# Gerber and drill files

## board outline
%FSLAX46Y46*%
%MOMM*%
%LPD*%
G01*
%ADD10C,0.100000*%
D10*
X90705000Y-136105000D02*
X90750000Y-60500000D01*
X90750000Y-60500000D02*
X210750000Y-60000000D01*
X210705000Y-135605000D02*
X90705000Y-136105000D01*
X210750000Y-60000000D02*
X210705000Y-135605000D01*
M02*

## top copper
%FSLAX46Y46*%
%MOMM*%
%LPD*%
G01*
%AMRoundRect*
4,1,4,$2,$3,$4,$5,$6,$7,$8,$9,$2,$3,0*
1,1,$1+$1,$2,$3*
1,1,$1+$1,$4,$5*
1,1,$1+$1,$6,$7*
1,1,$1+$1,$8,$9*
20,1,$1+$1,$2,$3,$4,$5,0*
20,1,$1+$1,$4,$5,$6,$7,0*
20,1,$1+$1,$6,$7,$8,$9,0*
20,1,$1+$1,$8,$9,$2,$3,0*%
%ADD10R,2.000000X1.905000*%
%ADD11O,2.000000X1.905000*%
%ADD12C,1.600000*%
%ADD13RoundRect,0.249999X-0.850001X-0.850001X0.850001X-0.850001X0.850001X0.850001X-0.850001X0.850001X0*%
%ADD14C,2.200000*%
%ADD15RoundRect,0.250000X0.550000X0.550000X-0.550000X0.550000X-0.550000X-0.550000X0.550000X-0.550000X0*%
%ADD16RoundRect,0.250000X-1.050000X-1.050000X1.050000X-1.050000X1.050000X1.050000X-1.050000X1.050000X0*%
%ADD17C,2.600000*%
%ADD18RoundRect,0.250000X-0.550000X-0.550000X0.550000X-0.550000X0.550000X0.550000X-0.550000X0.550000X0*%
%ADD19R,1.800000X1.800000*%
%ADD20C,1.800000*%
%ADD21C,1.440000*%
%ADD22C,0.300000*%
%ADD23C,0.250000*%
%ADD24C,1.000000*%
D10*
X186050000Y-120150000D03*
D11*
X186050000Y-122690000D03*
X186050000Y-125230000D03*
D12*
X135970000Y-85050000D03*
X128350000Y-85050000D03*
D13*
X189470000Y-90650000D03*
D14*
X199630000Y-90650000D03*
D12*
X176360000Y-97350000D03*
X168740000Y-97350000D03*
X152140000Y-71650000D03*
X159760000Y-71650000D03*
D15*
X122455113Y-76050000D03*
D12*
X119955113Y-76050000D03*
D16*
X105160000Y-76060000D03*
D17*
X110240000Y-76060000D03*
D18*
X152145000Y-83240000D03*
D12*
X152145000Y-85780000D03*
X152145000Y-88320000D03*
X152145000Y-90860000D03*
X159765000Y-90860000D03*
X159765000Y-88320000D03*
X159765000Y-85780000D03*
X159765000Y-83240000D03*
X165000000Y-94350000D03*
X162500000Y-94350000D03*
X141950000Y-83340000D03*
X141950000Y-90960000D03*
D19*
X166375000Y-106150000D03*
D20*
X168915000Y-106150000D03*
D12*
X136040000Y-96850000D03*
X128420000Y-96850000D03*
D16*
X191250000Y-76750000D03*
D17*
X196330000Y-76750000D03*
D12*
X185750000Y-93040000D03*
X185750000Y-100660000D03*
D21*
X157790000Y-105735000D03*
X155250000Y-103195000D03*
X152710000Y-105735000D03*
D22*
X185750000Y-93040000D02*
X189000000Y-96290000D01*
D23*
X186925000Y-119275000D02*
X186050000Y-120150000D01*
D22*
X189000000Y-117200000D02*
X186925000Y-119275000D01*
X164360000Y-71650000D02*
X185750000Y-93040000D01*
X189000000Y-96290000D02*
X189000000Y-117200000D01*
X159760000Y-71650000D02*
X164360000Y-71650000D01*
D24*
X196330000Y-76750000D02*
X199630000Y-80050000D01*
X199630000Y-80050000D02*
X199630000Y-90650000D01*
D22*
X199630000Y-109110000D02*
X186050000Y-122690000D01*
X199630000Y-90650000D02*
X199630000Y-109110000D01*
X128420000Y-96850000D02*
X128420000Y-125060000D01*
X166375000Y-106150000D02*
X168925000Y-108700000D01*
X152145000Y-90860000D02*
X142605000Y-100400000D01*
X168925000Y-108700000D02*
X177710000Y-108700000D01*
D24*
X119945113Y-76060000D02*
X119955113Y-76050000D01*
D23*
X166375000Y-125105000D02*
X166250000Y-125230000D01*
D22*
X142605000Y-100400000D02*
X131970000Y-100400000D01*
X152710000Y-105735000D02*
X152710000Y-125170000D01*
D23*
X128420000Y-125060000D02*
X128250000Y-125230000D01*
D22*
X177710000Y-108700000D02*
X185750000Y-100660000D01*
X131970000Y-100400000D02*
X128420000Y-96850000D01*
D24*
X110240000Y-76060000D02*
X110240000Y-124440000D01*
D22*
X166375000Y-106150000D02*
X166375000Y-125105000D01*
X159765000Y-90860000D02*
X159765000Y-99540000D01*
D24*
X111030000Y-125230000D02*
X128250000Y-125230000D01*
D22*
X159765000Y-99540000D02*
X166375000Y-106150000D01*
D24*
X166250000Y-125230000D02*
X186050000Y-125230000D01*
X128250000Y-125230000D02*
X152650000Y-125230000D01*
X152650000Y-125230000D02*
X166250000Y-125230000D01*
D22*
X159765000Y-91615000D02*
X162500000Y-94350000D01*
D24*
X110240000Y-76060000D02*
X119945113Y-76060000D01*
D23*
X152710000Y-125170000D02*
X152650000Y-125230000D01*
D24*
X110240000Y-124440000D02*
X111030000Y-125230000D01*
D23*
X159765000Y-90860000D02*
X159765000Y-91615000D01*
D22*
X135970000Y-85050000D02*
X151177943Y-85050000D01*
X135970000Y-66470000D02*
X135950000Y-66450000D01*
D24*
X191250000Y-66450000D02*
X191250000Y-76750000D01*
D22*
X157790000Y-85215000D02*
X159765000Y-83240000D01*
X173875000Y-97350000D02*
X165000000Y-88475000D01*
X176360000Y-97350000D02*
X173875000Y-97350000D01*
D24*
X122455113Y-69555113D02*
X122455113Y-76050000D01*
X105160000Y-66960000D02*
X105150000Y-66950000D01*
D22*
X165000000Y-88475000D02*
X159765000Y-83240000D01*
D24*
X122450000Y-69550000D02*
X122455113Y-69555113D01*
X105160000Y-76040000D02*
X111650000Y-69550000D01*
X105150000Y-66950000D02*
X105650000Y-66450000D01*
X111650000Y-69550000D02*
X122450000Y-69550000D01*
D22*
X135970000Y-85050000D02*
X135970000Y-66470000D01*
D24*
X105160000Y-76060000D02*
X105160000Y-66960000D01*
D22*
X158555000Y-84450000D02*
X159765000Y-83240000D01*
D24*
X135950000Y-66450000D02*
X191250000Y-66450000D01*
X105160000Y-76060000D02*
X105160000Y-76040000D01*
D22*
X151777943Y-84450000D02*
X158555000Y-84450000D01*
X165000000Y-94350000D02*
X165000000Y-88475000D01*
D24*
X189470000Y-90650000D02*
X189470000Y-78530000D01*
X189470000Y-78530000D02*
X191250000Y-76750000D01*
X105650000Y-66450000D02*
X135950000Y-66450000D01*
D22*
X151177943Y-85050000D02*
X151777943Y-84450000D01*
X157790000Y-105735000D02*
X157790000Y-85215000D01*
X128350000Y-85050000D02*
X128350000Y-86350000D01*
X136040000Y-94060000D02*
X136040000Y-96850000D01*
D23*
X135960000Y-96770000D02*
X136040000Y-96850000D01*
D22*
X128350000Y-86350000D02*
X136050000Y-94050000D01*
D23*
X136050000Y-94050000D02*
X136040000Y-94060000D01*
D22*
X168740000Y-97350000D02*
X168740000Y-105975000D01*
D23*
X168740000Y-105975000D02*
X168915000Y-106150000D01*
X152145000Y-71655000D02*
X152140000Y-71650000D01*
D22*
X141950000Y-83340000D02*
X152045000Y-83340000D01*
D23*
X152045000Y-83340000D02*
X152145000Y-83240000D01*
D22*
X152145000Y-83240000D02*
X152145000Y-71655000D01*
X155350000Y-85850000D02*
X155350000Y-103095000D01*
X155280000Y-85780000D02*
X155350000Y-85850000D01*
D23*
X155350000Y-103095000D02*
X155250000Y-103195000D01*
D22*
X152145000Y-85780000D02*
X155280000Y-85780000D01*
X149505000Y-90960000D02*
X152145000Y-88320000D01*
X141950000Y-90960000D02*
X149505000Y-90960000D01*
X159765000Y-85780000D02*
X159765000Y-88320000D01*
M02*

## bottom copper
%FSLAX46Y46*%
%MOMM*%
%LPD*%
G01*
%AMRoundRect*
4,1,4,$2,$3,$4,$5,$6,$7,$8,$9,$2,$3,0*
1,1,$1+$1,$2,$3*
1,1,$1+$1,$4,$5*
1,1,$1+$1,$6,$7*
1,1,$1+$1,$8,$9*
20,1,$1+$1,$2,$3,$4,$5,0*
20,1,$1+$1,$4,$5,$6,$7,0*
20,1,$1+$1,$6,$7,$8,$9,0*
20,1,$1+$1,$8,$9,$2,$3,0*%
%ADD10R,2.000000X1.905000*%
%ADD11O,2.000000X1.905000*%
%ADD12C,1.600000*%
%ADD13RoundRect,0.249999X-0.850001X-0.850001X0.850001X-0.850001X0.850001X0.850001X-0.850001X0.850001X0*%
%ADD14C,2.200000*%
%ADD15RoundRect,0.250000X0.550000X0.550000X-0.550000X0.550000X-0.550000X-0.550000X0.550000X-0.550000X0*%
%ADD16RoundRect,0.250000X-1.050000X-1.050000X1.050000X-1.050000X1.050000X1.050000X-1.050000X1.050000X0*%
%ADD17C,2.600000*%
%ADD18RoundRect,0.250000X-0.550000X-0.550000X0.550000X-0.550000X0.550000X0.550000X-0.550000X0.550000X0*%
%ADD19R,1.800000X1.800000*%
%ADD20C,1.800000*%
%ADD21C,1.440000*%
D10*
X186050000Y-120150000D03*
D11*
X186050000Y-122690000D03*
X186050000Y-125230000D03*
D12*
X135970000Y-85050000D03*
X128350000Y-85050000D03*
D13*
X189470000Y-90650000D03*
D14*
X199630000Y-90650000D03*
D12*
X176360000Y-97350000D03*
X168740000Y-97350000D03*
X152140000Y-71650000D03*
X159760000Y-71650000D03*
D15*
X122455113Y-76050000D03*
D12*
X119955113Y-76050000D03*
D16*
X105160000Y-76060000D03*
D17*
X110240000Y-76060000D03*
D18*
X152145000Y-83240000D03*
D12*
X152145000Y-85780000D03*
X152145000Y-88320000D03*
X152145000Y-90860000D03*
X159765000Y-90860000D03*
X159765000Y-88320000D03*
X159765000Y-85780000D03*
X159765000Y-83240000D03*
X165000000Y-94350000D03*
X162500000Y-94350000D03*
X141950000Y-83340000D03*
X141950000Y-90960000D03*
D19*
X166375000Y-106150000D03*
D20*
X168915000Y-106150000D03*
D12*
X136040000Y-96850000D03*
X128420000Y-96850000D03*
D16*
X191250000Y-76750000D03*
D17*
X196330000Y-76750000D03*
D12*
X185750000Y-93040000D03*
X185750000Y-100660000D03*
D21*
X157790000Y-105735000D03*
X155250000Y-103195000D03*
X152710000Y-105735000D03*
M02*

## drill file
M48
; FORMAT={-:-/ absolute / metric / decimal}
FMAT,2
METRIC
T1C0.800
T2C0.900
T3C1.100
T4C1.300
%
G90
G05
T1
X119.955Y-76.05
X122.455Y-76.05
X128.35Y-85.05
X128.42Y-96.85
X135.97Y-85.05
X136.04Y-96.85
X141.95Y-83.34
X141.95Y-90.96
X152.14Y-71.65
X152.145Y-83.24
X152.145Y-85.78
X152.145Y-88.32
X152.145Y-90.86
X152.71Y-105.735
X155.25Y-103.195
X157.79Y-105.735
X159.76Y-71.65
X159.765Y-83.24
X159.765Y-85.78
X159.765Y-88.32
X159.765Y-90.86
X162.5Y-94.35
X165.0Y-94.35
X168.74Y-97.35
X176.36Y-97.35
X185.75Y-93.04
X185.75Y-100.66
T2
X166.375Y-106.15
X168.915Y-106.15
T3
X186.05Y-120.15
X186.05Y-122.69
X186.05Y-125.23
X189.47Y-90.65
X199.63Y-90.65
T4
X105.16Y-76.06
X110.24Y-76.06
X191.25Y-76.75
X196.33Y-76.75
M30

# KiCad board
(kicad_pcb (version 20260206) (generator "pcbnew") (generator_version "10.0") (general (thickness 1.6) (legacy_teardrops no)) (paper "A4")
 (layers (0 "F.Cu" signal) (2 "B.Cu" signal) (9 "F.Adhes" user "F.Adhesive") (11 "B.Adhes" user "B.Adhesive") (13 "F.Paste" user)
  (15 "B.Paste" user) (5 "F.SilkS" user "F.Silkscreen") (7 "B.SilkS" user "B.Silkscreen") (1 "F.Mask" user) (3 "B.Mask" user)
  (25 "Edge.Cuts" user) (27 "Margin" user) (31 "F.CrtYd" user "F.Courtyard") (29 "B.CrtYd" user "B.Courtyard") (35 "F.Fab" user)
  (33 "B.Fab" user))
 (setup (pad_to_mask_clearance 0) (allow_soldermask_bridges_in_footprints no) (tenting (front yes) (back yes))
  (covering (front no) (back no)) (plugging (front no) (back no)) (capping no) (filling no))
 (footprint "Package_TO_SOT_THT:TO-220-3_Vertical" (layer "F.Cu") (at 186.05 120.15 -90)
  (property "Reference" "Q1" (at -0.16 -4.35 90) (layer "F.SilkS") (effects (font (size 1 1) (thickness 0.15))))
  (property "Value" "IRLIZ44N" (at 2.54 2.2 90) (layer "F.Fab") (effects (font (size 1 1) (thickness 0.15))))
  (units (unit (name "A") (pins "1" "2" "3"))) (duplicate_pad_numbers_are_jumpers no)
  (pad "1" thru_hole rect (at 0 0 270) (size 1.905 2) (drill 1.1) (layers "*.Cu" "*.Mask") (remove_unused_layers no) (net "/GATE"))
  (pad "2" thru_hole oval (at 2.54 0 270) (size 1.905 2) (drill 1.1) (layers "*.Cu" "*.Mask") (remove_unused_layers no) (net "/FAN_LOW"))
  (pad "3" thru_hole oval (at 5.08 0 270) (size 1.905 2) (drill 1.1) (layers "*.Cu" "*.Mask") (remove_unused_layers no) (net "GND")))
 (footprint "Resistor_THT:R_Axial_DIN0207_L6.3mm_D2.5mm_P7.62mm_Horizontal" (layer "F.Cu") (at 135.97 85.05 180)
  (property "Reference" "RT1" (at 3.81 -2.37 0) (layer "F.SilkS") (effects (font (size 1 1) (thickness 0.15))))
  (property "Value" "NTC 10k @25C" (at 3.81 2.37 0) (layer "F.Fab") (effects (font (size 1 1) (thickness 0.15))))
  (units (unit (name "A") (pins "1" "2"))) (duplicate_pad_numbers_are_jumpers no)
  (pad "1" thru_hole circle (at 0 0 180) (size 1.6 1.6) (drill 0.8) (layers "*.Cu" "*.Mask") (remove_unused_layers no) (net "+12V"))
  (pad "2" thru_hole circle (at 7.62 0 180) (size 1.6 1.6) (drill 0.8) (layers "*.Cu" "*.Mask") (remove_unused_layers no)
   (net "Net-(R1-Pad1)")))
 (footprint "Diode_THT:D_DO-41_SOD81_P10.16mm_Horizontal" (layer "F.Cu") (at 189.47 90.65)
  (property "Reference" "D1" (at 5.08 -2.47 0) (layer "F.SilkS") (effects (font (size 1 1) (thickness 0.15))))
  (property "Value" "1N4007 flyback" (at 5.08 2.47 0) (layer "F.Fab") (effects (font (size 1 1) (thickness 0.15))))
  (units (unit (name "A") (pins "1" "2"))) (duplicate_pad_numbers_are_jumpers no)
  (pad "1" thru_hole roundrect (at 0 0) (size 2.2 2.2) (drill 1.1) (layers "*.Cu" "*.Mask") (remove_unused_layers no)
   (roundrect_rratio 0.113636) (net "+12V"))
  (pad "2" thru_hole circle (at 10.16 0) (size 2.2 2.2) (drill 1.1) (layers "*.Cu" "*.Mask") (remove_unused_layers no) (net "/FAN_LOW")))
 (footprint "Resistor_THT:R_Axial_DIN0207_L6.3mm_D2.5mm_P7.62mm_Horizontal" (layer "F.Cu") (at 176.36 97.35 180)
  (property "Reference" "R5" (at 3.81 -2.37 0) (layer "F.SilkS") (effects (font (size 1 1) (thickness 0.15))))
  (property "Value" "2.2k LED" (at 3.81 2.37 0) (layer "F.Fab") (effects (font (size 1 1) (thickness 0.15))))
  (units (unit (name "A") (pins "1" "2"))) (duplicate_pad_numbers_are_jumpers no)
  (pad "1" thru_hole circle (at 0 0 180) (size 1.6 1.6) (drill 0.8) (layers "*.Cu" "*.Mask") (remove_unused_layers no) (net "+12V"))
  (pad "2" thru_hole circle (at 7.62 0 180) (size 1.6 1.6) (drill 0.8) (layers "*.Cu" "*.Mask") (remove_unused_layers no) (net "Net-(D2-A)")))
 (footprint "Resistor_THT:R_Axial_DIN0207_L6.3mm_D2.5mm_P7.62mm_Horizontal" (layer "F.Cu") (at 152.14 71.65)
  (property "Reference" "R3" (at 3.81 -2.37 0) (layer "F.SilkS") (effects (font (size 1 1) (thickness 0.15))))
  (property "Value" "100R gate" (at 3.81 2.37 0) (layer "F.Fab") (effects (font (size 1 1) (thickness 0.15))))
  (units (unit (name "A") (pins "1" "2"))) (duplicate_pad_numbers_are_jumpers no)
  (pad "1" thru_hole circle (at 0 0) (size 1.6 1.6) (drill 0.8) (layers "*.Cu" "*.Mask") (remove_unused_layers no) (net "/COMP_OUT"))
  (pad "2" thru_hole circle (at 7.62 0) (size 1.6 1.6) (drill 0.8) (layers "*.Cu" "*.Mask") (remove_unused_layers no) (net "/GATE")))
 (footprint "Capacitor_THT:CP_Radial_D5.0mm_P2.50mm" (layer "F.Cu") (at 122.455113 76.05 180)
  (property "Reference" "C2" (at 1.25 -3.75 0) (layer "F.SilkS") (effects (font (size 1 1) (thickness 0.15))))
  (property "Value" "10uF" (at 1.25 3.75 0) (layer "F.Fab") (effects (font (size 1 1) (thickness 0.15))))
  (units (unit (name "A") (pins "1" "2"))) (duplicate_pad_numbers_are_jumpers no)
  (pad "1" thru_hole roundrect (at 0 0 180) (size 1.6 1.6) (drill 0.8) (layers "*.Cu" "*.Mask") (remove_unused_layers no)
   (roundrect_rratio 0.15625) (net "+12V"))
  (pad "2" thru_hole circle (at 2.5 0 180) (size 1.6 1.6) (drill 0.8) (layers "*.Cu" "*.Mask") (remove_unused_layers no) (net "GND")))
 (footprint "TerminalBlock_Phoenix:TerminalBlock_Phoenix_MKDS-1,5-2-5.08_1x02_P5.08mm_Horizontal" (layer "F.Cu") (at 105.16 76.06)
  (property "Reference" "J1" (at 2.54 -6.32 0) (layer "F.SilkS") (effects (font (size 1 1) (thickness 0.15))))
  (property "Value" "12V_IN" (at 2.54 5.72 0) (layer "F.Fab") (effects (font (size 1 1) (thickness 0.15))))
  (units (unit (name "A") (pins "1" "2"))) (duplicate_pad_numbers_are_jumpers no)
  (pad "1" thru_hole roundrect (at 0 0) (size 2.6 2.6) (drill 1.3) (layers "*.Cu" "*.Mask") (remove_unused_layers no)
   (roundrect_rratio 0.096154) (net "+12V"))
  (pad "2" thru_hole circle (at 5.08 0) (size 2.6 2.6) (drill 1.3) (layers "*.Cu" "*.Mask") (remove_unused_layers no) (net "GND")))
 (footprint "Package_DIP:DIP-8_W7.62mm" (layer "F.Cu") (at 152.145 83.24)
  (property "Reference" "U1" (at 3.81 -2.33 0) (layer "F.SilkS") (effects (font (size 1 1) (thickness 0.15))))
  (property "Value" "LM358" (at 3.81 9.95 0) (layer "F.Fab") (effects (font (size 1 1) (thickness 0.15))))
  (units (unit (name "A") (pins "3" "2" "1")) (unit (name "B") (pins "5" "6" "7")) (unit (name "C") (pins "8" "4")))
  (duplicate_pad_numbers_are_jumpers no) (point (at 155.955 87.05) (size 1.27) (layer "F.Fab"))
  (pad "1" thru_hole roundrect (at 0 0) (size 1.6 1.6) (drill 0.8) (layers "*.Cu" "*.Mask") (remove_unused_layers no)
   (roundrect_rratio 0.15625) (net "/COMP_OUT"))
  (pad "2" thru_hole circle (at 0 2.54) (size 1.6 1.6) (drill 0.8) (layers "*.Cu" "*.Mask") (remove_unused_layers no) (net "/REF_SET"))
  (pad "3" thru_hole circle (at 0 5.08) (size 1.6 1.6) (drill 0.8) (layers "*.Cu" "*.Mask") (remove_unused_layers no) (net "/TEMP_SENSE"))
  (pad "4" thru_hole circle (at 0 7.62) (size 1.6 1.6) (drill 0.8) (layers "*.Cu" "*.Mask") (remove_unused_layers no) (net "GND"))
  (pad "5" thru_hole circle (at 7.62 7.62) (size 1.6 1.6) (drill 0.8) (layers "*.Cu" "*.Mask") (remove_unused_layers no) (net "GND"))
  (pad "6" thru_hole circle (at 7.62 5.08) (size 1.6 1.6) (drill 0.8) (layers "*.Cu" "*.Mask") (remove_unused_layers no) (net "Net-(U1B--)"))
  (pad "7" thru_hole circle (at 7.62 2.54) (size 1.6 1.6) (drill 0.8) (layers "*.Cu" "*.Mask") (remove_unused_layers no) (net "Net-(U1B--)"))
  (pad "8" thru_hole circle (at 7.62 0) (size 1.6 1.6) (drill 0.8) (layers "*.Cu" "*.Mask") (remove_unused_layers no) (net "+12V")))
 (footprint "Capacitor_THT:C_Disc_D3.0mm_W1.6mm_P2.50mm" (layer "F.Cu") (at 165 94.35 180)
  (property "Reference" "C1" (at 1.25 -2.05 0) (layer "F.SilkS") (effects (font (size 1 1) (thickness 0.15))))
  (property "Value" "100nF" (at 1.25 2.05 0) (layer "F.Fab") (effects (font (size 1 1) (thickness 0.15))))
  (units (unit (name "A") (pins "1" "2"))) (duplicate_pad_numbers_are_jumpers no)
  (pad "1" thru_hole circle (at 0 0 180) (size 1.6 1.6) (drill 0.8) (layers "*.Cu" "*.Mask") (remove_unused_layers no) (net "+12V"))
  (pad "2" thru_hole circle (at 2.5 0 180) (size 1.6 1.6) (drill 0.8) (layers "*.Cu" "*.Mask") (remove_unused_layers no) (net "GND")))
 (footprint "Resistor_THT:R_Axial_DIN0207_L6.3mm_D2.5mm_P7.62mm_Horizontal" (layer "F.Cu") (at 141.95 83.34 -90)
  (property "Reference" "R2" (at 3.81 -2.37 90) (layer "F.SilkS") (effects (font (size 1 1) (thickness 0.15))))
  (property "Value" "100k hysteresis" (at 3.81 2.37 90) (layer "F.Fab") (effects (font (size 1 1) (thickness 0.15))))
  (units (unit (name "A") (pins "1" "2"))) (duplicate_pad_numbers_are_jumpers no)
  (pad "1" thru_hole circle (at 0 0 270) (size 1.6 1.6) (drill 0.8) (layers "*.Cu" "*.Mask") (remove_unused_layers no) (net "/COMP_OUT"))
  (pad "2" thru_hole circle (at 7.62 0 270) (size 1.6 1.6) (drill 0.8) (layers "*.Cu" "*.Mask") (remove_unused_layers no)
   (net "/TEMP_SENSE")))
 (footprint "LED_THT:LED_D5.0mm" (layer "F.Cu") (at 166.375 106.15)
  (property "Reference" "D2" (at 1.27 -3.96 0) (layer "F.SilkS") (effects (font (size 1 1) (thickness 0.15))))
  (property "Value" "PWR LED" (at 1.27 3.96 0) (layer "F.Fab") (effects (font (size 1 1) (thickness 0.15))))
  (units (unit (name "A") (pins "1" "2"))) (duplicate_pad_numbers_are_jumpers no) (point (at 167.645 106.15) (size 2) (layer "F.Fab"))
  (pad "1" thru_hole rect (at 0 0) (size 1.8 1.8) (drill 0.9) (layers "*.Cu" "*.Mask") (remove_unused_layers no) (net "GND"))
  (pad "2" thru_hole circle (at 2.54 0) (size 1.8 1.8) (drill 0.9) (layers "*.Cu" "*.Mask") (remove_unused_layers no) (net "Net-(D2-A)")))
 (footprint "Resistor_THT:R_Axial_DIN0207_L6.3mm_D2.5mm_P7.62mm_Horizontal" (layer "F.Cu") (at 136.04 96.85 180)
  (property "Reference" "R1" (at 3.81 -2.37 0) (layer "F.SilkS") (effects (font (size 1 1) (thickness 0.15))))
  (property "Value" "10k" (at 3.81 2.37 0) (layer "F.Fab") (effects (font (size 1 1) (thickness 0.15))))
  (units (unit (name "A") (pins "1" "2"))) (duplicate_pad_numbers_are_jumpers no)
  (pad "1" thru_hole circle (at 0 0 180) (size 1.6 1.6) (drill 0.8) (layers "*.Cu" "*.Mask") (remove_unused_layers no) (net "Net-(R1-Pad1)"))
  (pad "2" thru_hole circle (at 7.62 0 180) (size 1.6 1.6) (drill 0.8) (layers "*.Cu" "*.Mask") (remove_unused_layers no) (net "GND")))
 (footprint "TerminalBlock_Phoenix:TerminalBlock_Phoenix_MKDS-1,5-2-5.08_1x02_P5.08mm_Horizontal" (layer "F.Cu") (at 191.25 76.75)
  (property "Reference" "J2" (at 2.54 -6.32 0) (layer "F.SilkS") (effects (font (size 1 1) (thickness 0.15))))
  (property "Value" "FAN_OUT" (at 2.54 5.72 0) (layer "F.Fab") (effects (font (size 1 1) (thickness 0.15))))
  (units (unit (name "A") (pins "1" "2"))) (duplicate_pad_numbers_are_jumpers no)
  (pad "1" thru_hole roundrect (at 0 0) (size 2.6 2.6) (drill 1.3) (layers "*.Cu" "*.Mask") (remove_unused_layers no)
   (roundrect_rratio 0.096154) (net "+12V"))
  (pad "2" thru_hole circle (at 5.08 0) (size 2.6 2.6) (drill 1.3) (layers "*.Cu" "*.Mask") (remove_unused_layers no) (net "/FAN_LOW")))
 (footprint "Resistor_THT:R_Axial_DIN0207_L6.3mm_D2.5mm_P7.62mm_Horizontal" (layer "F.Cu") (at 185.75 93.04 -90)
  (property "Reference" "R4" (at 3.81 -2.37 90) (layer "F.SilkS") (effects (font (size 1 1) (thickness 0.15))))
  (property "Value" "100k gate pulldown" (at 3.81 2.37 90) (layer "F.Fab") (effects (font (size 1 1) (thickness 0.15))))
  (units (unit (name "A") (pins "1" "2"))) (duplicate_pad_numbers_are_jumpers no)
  (pad "1" thru_hole circle (at 0 0 270) (size 1.6 1.6) (drill 0.8) (layers "*.Cu" "*.Mask") (remove_unused_layers no) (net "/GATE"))
  (pad "2" thru_hole circle (at 7.62 0 270) (size 1.6 1.6) (drill 0.8) (layers "*.Cu" "*.Mask") (remove_unused_layers no) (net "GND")))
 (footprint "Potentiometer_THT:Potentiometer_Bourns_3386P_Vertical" (layer "F.Cu") (at 157.79 105.735 90)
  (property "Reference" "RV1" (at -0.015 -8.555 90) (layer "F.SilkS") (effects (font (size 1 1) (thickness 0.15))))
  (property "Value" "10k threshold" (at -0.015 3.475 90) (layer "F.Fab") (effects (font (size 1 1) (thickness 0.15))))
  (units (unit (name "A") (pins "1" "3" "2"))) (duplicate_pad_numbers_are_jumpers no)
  (pad "1" thru_hole circle (at 0 0 90) (size 1.44 1.44) (drill 0.8) (layers "*.Cu" "*.Mask") (remove_unused_layers no) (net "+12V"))
  (pad "2" thru_hole circle (at 2.54 -2.54 90) (size 1.44 1.44) (drill 0.8) (layers "*.Cu" "*.Mask") (remove_unused_layers no)
   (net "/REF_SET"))
  (pad "3" thru_hole circle (at 0 -5.08 90) (size 1.44 1.44) (drill 0.8) (layers "*.Cu" "*.Mask") (remove_unused_layers no) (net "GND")))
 (gr_line (start 90.705 136.105) (end 90.75 60.5) (stroke (width 0.1) (type solid)) (layer "Edge.Cuts"))
 (gr_line (start 90.75 60.5) (end 210.75 60) (stroke (width 0.1) (type solid)) (layer "Edge.Cuts"))
 (gr_line (start 210.705 135.605) (end 90.705 136.105) (stroke (width 0.1) (type solid)) (layer "Edge.Cuts"))
 (gr_line (start 210.75 60) (end 210.705 135.605) (stroke (width 0.1) (type solid)) (layer "Edge.Cuts"))
 (segment (start 185.75 93.04) (end 189 96.29) (width 0.3) (layer "F.Cu") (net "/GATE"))
 (segment (start 186.925 119.275) (end 186.05 120.15) (width 0.25) (layer "F.Cu") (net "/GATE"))
 (segment (start 189 117.2) (end 186.925 119.275) (width 0.3) (layer "F.Cu") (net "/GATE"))
 (segment (start 164.36 71.65) (end 185.75 93.04) (width 0.3) (layer "F.Cu") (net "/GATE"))
 (segment (start 189 96.29) (end 189 117.2) (width 0.3) (layer "F.Cu") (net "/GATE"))
 (segment (start 159.76 71.65) (end 164.36 71.65) (width 0.3) (layer "F.Cu") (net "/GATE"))
 (segment (start 196.33 76.75) (end 199.63 80.05) (width 1) (layer "F.Cu") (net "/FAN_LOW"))
 (segment (start 199.63 80.05) (end 199.63 90.65) (width 1) (layer "F.Cu") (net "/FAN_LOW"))
 (segment (start 199.63 109.11) (end 186.05 122.69) (width 0.3) (layer "F.Cu") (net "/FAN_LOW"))
 (segment (start 199.63 90.65) (end 199.63 109.11) (width 0.3) (layer "F.Cu") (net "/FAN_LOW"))
 (segment (start 128.42 96.85) (end 128.42 125.06) (width 0.3) (layer "F.Cu") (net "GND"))
 (segment (start 166.375 106.15) (end 168.925 108.7) (width 0.3) (layer "F.Cu") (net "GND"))
 (segment (start 152.145 90.86) (end 142.605 100.4) (width 0.3) (layer "F.Cu") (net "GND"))
 (segment (start 168.925 108.7) (end 177.71 108.7) (width 0.3) (layer "F.Cu") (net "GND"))
 (segment (start 119.945113 76.06) (end 119.955113 76.05) (width 1) (layer "F.Cu") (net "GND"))
 (segment (start 166.375 125.105) (end 166.25 125.23) (width 0.25) (layer "F.Cu") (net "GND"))
 (segment (start 142.605 100.4) (end 131.97 100.4) (width 0.3) (layer "F.Cu") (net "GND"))
 (segment (start 152.71 105.735) (end 152.71 125.17) (width 0.3) (layer "F.Cu") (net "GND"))
 (segment (start 128.42 125.06) (end 128.25 125.23) (width 0.25) (layer "F.Cu") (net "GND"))
 (segment (start 177.71 108.7) (end 185.75 100.66) (width 0.3) (layer "F.Cu") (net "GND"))
 (segment (start 131.97 100.4) (end 128.42 96.85) (width 0.3) (layer "F.Cu") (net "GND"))
 (segment (start 110.24 76.06) (end 110.24 124.44) (width 1) (layer "F.Cu") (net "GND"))
 (segment (start 166.375 106.15) (end 166.375 125.105) (width 0.3) (layer "F.Cu") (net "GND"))
 (segment (start 159.765 90.86) (end 159.765 99.54) (width 0.3) (layer "F.Cu") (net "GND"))
 (segment (start 111.03 125.23) (end 128.25 125.23) (width 1) (layer "F.Cu") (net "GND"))
 (segment (start 159.765 99.54) (end 166.375 106.15) (width 0.3) (layer "F.Cu") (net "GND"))
 (segment (start 166.25 125.23) (end 186.05 125.23) (width 1) (layer "F.Cu") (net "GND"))
 (segment (start 128.25 125.23) (end 152.65 125.23) (width 1) (layer "F.Cu") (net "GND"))
 (segment (start 152.65 125.23) (end 166.25 125.23) (width 1) (layer "F.Cu") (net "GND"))
 (segment (start 159.765 91.615) (end 162.5 94.35) (width 0.3) (layer "F.Cu") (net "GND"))
 (segment (start 110.24 76.06) (end 119.945113 76.06) (width 1) (layer "F.Cu") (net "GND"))
 (segment (start 152.71 125.17) (end 152.65 125.23) (width 0.25) (layer "F.Cu") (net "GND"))
 (segment (start 110.24 124.44) (end 111.03 125.23) (width 1) (layer "F.Cu") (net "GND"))
 (segment (start 159.765 90.86) (end 159.765 91.615) (width 0.25) (layer "F.Cu") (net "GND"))
 (segment (start 135.97 85.05) (end 151.177943 85.05) (width 0.3) (layer "F.Cu") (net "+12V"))
 (segment (start 135.97 66.47) (end 135.95 66.45) (width 0.3) (layer "F.Cu") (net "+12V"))
 (segment (start 191.25 66.45) (end 191.25 76.75) (width 1) (layer "F.Cu") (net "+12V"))
 (segment (start 157.79 85.215) (end 159.765 83.24) (width 0.3) (layer "F.Cu") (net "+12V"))
 (segment (start 173.875 97.35) (end 165 88.475) (width 0.3) (layer "F.Cu") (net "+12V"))
 (segment (start 176.36 97.35) (end 173.875 97.35) (width 0.3) (layer "F.Cu") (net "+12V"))
 (segment (start 122.455113 69.555113) (end 122.455113 76.05) (width 1) (layer "F.Cu") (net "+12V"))
 (segment (start 105.16 66.96) (end 105.15 66.95) (width 1) (layer "F.Cu") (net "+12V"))
 (segment (start 165 88.475) (end 159.765 83.24) (width 0.3) (layer "F.Cu") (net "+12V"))
 (segment (start 122.45 69.55) (end 122.455113 69.555113) (width 1) (layer "F.Cu") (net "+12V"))
 (segment (start 105.16 76.04) (end 111.65 69.55) (width 1) (layer "F.Cu") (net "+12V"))
 (segment (start 105.15 66.95) (end 105.65 66.45) (width 1) (layer "F.Cu") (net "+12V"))
 (segment (start 111.65 69.55) (end 122.45 69.55) (width 1) (layer "F.Cu") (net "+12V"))
 (segment (start 135.97 85.05) (end 135.97 66.47) (width 0.3) (layer "F.Cu") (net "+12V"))
 (segment (start 105.16 76.06) (end 105.16 66.96) (width 1) (layer "F.Cu") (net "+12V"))
 (segment (start 158.555 84.45) (end 159.765 83.24) (width 0.3) (layer "F.Cu") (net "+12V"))
 (segment (start 135.95 66.45) (end 191.25 66.45) (width 1) (layer "F.Cu") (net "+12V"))
 (segment (start 105.16 76.06) (end 105.16 76.04) (width 1) (layer "F.Cu") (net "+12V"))
 (segment (start 151.777943 84.45) (end 158.555 84.45) (width 0.3) (layer "F.Cu") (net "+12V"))
 (segment (start 165 94.35) (end 165 88.475) (width 0.3) (layer "F.Cu") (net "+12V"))
 (segment (start 189.47 90.65) (end 189.47 78.53) (width 1) (layer "F.Cu") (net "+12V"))
 (segment (start 189.47 78.53) (end 191.25 76.75) (width 1) (layer "F.Cu") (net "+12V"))
 (segment (start 105.65 66.45) (end 135.95 66.45) (width 1) (layer "F.Cu") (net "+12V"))
 (segment (start 151.177943 85.05) (end 151.777943 84.45) (width 0.3) (layer "F.Cu") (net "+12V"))
 (segment (start 157.79 105.735) (end 157.79 85.215) (width 0.3) (layer "F.Cu") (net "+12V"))
 (segment (start 128.35 85.05) (end 128.35 86.35) (width 0.3) (layer "F.Cu") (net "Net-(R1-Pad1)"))
 (segment (start 136.04 94.06) (end 136.04 96.85) (width 0.3) (layer "F.Cu") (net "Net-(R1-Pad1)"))
 (segment (start 135.96 96.77) (end 136.04 96.85) (width 0.25) (layer "F.Cu") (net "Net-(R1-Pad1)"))
 (segment (start 128.35 86.35) (end 136.05 94.05) (width 0.3) (layer "F.Cu") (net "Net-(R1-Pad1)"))
 (segment (start 136.05 94.05) (end 136.04 94.06) (width 0.25) (layer "F.Cu") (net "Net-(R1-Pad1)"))
 (segment (start 168.74 97.35) (end 168.74 105.975) (width 0.3) (layer "F.Cu") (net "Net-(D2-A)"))
 (segment (start 168.74 105.975) (end 168.915 106.15) (width 0.25) (layer "F.Cu") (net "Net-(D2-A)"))
 (segment (start 152.145 71.655) (end 152.14 71.65) (width 0.25) (layer "F.Cu") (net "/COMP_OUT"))
 (segment (start 141.95 83.34) (end 152.045 83.34) (width 0.3) (layer "F.Cu") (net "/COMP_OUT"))
 (segment (start 152.045 83.34) (end 152.145 83.24) (width 0.25) (layer "F.Cu") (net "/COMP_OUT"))
 (segment (start 152.145 83.24) (end 152.145 71.655) (width 0.3) (layer "F.Cu") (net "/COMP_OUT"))
 (segment (start 155.35 85.85) (end 155.35 103.095) (width 0.3) (layer "F.Cu") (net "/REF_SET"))
 (segment (start 155.28 85.78) (end 155.35 85.85) (width 0.3) (layer "F.Cu") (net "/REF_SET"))
 (segment (start 155.35 103.095) (end 155.25 103.195) (width 0.25) (layer "F.Cu") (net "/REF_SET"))
 (segment (start 152.145 85.78) (end 155.28 85.78) (width 0.3) (layer "F.Cu") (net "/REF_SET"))
 (segment (start 149.505 90.96) (end 152.145 88.32) (width 0.3) (layer "F.Cu") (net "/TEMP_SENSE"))
 (segment (start 141.95 90.96) (end 149.505 90.96) (width 0.3) (layer "F.Cu") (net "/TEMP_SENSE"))
 (segment (start 159.765 85.78) (end 159.765 88.32) (width 0.3) (layer "F.Cu") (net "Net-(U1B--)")))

